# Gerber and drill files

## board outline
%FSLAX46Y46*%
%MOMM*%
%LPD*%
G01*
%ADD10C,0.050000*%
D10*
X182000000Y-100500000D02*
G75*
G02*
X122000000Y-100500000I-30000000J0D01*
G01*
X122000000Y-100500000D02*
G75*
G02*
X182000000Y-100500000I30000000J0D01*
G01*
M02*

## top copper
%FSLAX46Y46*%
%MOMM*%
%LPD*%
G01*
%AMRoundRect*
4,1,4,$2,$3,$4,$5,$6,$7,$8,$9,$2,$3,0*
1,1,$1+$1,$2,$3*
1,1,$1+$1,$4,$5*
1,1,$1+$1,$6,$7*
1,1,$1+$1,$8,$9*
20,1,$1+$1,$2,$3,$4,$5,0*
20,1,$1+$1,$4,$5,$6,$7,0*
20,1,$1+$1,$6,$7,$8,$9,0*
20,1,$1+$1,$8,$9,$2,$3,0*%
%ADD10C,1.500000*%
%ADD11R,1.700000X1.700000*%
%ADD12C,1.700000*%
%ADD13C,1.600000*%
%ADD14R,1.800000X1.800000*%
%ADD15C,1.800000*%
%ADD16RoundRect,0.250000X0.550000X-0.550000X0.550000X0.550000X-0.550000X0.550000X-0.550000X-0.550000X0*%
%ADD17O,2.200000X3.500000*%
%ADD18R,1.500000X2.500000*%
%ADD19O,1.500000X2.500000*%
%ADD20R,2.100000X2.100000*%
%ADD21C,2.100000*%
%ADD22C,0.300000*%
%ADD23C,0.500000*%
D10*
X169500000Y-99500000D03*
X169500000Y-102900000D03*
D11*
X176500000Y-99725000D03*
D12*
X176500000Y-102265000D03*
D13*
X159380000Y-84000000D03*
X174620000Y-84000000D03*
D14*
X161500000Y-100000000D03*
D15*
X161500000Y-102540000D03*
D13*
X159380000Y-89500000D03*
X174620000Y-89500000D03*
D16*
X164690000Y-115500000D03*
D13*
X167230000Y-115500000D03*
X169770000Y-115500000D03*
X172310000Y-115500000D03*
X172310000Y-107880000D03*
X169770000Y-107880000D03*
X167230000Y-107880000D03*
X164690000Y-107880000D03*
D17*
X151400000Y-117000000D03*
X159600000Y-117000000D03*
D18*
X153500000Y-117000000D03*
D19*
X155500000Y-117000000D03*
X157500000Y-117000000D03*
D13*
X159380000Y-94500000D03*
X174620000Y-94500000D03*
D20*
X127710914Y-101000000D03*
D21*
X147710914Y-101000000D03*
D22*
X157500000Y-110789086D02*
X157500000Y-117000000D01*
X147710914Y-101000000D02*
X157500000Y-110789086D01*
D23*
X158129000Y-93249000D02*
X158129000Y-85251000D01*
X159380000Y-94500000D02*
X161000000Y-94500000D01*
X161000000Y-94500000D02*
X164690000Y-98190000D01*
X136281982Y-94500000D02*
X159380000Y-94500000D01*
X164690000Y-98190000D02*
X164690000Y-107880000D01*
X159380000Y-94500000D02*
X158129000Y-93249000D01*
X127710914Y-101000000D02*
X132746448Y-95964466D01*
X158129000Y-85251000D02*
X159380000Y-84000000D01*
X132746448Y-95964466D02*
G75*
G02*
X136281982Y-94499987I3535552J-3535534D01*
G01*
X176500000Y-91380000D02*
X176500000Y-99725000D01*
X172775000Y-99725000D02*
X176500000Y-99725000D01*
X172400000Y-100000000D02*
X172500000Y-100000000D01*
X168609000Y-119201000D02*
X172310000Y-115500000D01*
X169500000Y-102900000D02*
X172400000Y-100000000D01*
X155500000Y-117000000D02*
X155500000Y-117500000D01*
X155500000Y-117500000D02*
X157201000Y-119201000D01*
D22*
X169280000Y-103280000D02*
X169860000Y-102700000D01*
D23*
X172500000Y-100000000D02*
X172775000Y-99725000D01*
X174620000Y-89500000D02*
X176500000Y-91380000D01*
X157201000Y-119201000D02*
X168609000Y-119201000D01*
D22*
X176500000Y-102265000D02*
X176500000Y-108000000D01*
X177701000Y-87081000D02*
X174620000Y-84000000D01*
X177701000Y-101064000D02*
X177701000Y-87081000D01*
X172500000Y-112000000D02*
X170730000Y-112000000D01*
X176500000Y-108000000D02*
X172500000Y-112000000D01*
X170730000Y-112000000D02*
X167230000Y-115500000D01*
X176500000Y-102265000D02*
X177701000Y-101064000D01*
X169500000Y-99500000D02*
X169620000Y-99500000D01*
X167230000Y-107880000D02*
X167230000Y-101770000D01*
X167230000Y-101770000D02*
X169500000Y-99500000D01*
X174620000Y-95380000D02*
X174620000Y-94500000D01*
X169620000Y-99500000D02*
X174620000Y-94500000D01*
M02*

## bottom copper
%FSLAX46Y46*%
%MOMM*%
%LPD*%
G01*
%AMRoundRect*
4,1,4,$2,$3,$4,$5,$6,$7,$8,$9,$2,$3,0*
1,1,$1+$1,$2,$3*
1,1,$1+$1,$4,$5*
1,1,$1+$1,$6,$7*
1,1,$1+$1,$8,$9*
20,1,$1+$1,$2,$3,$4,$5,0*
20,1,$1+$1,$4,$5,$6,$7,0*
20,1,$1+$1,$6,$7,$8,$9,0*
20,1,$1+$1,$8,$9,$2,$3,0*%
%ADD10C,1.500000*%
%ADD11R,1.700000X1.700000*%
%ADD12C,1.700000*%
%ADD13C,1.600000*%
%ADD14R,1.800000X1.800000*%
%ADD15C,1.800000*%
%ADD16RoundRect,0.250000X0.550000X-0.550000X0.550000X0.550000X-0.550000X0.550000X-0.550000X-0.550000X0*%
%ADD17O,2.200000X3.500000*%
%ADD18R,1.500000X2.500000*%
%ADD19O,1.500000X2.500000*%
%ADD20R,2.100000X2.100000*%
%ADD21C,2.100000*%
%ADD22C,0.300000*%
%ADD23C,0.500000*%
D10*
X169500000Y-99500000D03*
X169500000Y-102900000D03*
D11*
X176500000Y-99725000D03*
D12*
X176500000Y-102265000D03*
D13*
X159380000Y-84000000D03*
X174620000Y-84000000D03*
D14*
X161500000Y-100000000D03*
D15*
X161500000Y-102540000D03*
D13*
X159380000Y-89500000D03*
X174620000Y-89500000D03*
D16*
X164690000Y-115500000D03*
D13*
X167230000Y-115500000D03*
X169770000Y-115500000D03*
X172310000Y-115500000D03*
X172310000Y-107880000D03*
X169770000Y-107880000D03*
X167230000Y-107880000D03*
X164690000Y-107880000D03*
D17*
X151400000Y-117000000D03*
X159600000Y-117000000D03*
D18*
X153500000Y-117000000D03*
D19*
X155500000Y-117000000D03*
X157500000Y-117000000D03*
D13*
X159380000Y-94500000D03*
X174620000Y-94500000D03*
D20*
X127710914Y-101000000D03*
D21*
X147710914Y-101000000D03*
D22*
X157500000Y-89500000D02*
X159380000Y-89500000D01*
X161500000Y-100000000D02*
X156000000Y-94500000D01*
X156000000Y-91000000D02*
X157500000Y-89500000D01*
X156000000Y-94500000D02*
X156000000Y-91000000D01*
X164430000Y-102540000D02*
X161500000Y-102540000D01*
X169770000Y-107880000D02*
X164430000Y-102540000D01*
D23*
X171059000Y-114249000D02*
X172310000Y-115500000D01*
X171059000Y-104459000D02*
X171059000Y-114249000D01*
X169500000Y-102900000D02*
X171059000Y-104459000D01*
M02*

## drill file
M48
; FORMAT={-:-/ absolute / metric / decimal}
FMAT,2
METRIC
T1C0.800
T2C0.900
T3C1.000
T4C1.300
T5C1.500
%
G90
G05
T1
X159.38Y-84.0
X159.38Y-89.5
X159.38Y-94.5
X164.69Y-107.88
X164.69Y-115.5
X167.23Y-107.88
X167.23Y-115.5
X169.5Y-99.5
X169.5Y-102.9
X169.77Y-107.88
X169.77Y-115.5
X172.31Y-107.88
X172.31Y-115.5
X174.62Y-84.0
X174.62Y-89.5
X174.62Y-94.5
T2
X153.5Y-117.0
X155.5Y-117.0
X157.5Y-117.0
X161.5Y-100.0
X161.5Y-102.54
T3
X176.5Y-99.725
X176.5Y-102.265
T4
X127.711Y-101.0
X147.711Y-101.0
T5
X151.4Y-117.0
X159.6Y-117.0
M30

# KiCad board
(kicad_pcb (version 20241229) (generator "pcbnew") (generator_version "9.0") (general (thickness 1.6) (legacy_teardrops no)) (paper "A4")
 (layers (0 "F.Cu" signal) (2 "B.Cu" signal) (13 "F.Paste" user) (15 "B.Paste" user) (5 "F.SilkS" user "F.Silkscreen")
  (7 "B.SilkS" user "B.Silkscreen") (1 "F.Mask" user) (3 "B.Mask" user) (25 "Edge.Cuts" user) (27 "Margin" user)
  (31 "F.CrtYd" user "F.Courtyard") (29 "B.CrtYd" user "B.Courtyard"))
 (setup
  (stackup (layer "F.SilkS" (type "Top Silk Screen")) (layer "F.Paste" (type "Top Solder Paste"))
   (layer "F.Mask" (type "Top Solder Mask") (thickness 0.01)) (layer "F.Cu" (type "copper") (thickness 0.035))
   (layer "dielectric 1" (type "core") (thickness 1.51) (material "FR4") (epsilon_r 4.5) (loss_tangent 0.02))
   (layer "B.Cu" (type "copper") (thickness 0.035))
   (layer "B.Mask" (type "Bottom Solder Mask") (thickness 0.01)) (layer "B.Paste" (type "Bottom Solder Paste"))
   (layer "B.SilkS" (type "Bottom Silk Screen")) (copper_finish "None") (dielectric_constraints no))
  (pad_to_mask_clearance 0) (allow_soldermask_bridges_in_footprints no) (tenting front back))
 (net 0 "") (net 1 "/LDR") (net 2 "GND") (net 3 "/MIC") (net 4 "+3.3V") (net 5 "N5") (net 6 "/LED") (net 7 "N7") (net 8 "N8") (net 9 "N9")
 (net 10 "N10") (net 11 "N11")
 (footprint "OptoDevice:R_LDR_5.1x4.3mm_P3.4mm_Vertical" (layer "F.Cu") (at 169.5 99.5 -90)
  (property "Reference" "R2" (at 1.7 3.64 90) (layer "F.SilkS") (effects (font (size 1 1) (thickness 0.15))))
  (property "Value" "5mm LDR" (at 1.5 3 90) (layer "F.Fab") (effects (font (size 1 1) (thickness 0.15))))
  (pad "1" thru_hole circle (at 0 0 270) (size 1.5 1.5) (drill 0.8) (layers "*.Cu" "*.Mask") (remove_unused_layers no) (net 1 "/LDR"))
  (pad "2" thru_hole circle (at 3.4 0 270) (size 1.5 1.5) (drill 0.8) (layers "*.Cu" "*.Mask") (remove_unused_layers no) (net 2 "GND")))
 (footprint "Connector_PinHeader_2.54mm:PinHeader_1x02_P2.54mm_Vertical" (layer "F.Cu") (at 176.5 99.725)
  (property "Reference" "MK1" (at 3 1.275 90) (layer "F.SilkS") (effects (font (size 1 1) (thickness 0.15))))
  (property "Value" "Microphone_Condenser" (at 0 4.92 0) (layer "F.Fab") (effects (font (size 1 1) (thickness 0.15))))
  (pad "1" thru_hole rect (at 0 0) (size 1.7 1.7) (drill 1) (layers "*.Cu" "*.Mask") (remove_unused_layers no) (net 2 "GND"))
  (pad "2" thru_hole circle (at 0 2.54) (size 1.7 1.7) (drill 1) (layers "*.Cu" "*.Mask") (remove_unused_layers no) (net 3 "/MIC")))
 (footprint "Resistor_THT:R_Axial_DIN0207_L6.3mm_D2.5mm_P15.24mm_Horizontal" (layer "F.Cu") (at 159.38 84)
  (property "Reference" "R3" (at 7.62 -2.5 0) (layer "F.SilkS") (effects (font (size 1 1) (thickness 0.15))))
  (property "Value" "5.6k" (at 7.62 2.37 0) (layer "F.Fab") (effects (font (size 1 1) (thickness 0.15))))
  (pad "1" thru_hole circle (at 0 0) (size 1.6 1.6) (drill 0.8) (layers "*.Cu" "*.Mask") (remove_unused_layers no) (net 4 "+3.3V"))
  (pad "2" thru_hole circle (at 15.24 0) (size 1.6 1.6) (drill 0.8) (layers "*.Cu" "*.Mask") (remove_unused_layers no) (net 3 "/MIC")))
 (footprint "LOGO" (layer "F.Cu") (at 151.915435 78.764812)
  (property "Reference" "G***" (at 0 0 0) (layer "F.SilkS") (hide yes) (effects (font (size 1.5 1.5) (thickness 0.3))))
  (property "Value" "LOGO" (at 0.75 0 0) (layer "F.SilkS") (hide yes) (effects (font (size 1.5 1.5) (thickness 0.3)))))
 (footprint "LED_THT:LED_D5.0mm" (layer "F.Cu") (at 161.5 100 -90)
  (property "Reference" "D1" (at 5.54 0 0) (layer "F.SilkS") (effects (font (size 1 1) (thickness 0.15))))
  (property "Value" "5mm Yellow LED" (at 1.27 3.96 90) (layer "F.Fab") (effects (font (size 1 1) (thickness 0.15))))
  (pad "1" thru_hole rect (at 0 0 270) (size 1.8 1.8) (drill 0.9) (layers "*.Cu" "*.Mask") (remove_unused_layers no) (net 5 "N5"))
  (pad "2" thru_hole circle (at 2.54 0 270) (size 1.8 1.8) (drill 0.9) (layers "*.Cu" "*.Mask") (remove_unused_layers no) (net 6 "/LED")))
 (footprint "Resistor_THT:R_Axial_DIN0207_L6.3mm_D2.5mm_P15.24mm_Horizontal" (layer "F.Cu") (at 159.38 89.5)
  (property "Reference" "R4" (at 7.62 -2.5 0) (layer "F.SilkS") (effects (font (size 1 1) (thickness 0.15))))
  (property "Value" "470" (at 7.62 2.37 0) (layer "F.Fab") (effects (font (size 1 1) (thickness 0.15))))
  (pad "1" thru_hole circle (at 0 0) (size 1.6 1.6) (drill 0.8) (layers "*.Cu" "*.Mask") (remove_unused_layers no) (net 5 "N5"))
  (pad "2" thru_hole circle (at 15.24 0) (size 1.6 1.6) (drill 0.8) (layers "*.Cu" "*.Mask") (remove_unused_layers no) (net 2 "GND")))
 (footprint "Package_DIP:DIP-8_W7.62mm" (layer "F.Cu") (at 164.69 115.5 90)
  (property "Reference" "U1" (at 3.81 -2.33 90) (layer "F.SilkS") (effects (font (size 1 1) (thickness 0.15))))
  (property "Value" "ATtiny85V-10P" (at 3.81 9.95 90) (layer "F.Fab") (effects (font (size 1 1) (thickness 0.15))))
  (pad "1" thru_hole roundrect (at 0 0 90) (size 1.6 1.6) (drill 0.8) (layers "*.Cu" "*.Mask") (remove_unused_layers no)
   (roundrect_rratio 0.15625) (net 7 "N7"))
  (pad "2" thru_hole circle (at 0 2.54 90) (size 1.6 1.6) (drill 0.8) (layers "*.Cu" "*.Mask") (remove_unused_layers no) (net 3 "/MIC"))
  (pad "3" thru_hole circle (at 0 5.08 90) (size 1.6 1.6) (drill 0.8) (layers "*.Cu" "*.Mask") (remove_unused_layers no) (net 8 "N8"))
  (pad "4" thru_hole circle (at 0 7.62 90) (size 1.6 1.6) (drill 0.8) (layers "*.Cu" "*.Mask") (remove_unused_layers no) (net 2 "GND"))
  (pad "5" thru_hole circle (at 7.62 7.62 90) (size 1.6 1.6) (drill 0.8) (layers "*.Cu" "*.Mask") (remove_unused_layers no) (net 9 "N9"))
  (pad "6" thru_hole circle (at 7.62 5.08 90) (size 1.6 1.6) (drill 0.8) (layers "*.Cu" "*.Mask") (remove_unused_layers no) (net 6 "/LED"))
  (pad "7" thru_hole circle (at 7.62 2.54 90) (size 1.6 1.6) (drill 0.8) (layers "*.Cu" "*.Mask") (remove_unused_layers no) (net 1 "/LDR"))
  (pad "8" thru_hole circle (at 7.62 0 90) (size 1.6 1.6) (drill 0.8) (layers "*.Cu" "*.Mask") (remove_unused_layers no) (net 4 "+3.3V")))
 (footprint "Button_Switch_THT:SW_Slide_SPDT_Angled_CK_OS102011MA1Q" (layer "F.Cu") (at 153.5 117)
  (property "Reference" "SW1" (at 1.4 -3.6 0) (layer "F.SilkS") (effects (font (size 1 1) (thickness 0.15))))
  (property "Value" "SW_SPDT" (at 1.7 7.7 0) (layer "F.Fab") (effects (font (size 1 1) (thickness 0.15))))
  (pad "" thru_hole oval (at -2.1 0) (size 2.2 3.5) (drill 1.5) (layers "*.Cu" "*.Mask") (remove_unused_layers no))
  (pad "" thru_hole oval (at 6.1 0) (size 2.2 3.5) (drill 1.5) (layers "*.Cu" "*.Mask") (remove_unused_layers no))
  (pad "1" thru_hole rect (at 0 0) (size 1.5 2.5) (drill 0.9) (layers "*.Cu" "*.Mask") (remove_unused_layers no) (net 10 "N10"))
  (pad "2" thru_hole oval (at 2 0) (size 1.5 2.5) (drill 0.9) (layers "*.Cu" "*.Mask") (remove_unused_layers no) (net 2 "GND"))
  (pad "3" thru_hole oval (at 4 0) (size 1.5 2.5) (drill 0.9) (layers "*.Cu" "*.Mask") (remove_unused_layers no) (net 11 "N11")))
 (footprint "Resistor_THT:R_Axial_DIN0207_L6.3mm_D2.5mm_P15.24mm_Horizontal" (layer "F.Cu") (at 159.38 94.5)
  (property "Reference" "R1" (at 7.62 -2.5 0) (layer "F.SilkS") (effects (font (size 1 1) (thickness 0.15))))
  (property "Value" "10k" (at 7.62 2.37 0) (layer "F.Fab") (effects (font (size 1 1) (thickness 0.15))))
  (pad "1" thru_hole circle (at 0 0) (size 1.6 1.6) (drill 0.8) (layers "*.Cu" "*.Mask") (remove_unused_layers no) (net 4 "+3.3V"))
  (pad "2" thru_hole circle (at 15.24 0) (size 1.6 1.6) (drill 0.8) (layers "*.Cu" "*.Mask") (remove_unused_layers no) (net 1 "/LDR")))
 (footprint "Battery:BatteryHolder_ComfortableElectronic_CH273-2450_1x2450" (layer "F.Cu") (at 127.710914 101)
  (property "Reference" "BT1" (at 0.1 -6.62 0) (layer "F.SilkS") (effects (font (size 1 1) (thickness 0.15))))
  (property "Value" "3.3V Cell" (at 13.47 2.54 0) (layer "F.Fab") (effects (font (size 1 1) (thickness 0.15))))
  (pad "1" thru_hole rect (at 0 0 270) (size 2.1 2.1) (drill 1.3) (layers "*.Cu" "*.Mask") (remove_unused_layers no) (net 4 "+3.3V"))
  (pad "2" thru_hole circle (at 20 0 270) (size 2.1 2.1) (drill 1.3) (layers "*.Cu" "*.Mask") (remove_unused_layers no) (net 11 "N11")))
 (gr_circle (center 152 100.5) (end 182 100.5) (stroke (width 0.05) (type solid)) (fill no) (locked yes) (layer "Edge.Cuts"))
 (segment (start 157.5 110.789086) (end 157.5 117) (width 0.3) (layer "F.Cu") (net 11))
 (segment (start 147.710914 101) (end 157.5 110.789086) (width 0.3) (layer "F.Cu") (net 11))
 (segment (start 158.129 93.249) (end 158.129 85.251) (width 0.5) (layer "F.Cu") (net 4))
 (segment (start 159.38 94.5) (end 161 94.5) (width 0.5) (layer "F.Cu") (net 4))
 (segment (start 161 94.5) (end 164.69 98.19) (width 0.5) (layer "F.Cu") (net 4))
 (segment (start 136.281982 94.5) (end 159.38 94.5) (width 0.5) (layer "F.Cu") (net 4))
 (segment (start 164.69 98.19) (end 164.69 107.88) (width 0.5) (layer "F.Cu") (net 4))
 (segment (start 159.38 94.5) (end 158.129 93.249) (width 0.5) (layer "F.Cu") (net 4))
 (segment (start 127.710914 101) (end 132.746448 95.964466) (width 0.5) (layer "F.Cu") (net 4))
 (segment (start 158.129 85.251) (end 159.38 84) (width 0.5) (layer "F.Cu") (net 4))
 (arc (start 132.746448 95.964466) (mid 134.368565 94.880602) (end 136.281982 94.5) (width 0.5) (layer "F.Cu") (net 4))
 (segment (start 157.5 89.5) (end 159.38 89.5) (width 0.3) (layer "B.Cu") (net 5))
 (segment (start 161.5 100) (end 156 94.5) (width 0.3) (layer "B.Cu") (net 5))
 (segment (start 156 91) (end 157.5 89.5) (width 0.3) (layer "B.Cu") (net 5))
 (segment (start 156 94.5) (end 156 91) (width 0.3) (layer "B.Cu") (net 5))
 (segment (start 164.43 102.54) (end 161.5 102.54) (width 0.3) (layer "B.Cu") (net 6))
 (segment (start 169.77 107.88) (end 164.43 102.54) (width 0.3) (layer "B.Cu") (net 6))
 (segment (start 176.5 91.38) (end 176.5 99.725) (width 0.5) (layer "F.Cu") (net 2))
 (segment (start 172.775 99.725) (end 176.5 99.725) (width 0.5) (layer "F.Cu") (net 2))
 (segment (start 172.4 100) (end 172.5 100) (width 0.5) (layer "F.Cu") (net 2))
 (segment (start 168.609 119.201) (end 172.31 115.5) (width 0.5) (layer "F.Cu") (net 2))
 (segment (start 169.5 102.9) (end 172.4 100) (width 0.5) (layer "F.Cu") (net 2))
 (segment (start 155.5 117) (end 155.5 117.5) (width 0.5) (layer "F.Cu") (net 2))
 (segment (start 155.5 117.5) (end 157.201 119.201) (width 0.5) (layer "F.Cu") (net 2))
 (segment (start 169.28 103.28) (end 169.86 102.7) (width 0.3) (layer "F.Cu") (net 2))
 (segment (start 172.5 100) (end 172.775 99.725) (width 0.5) (layer "F.Cu") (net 2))
 (segment (start 174.62 89.5) (end 176.5 91.38) (width 0.5) (layer "F.Cu") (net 2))
 (segment (start 157.201 119.201) (end 168.609 119.201) (width 0.5) (layer "F.Cu") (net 2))
 (segment (start 171.059 114.249) (end 172.31 115.5) (width 0.5) (layer "B.Cu") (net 2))
 (segment (start 171.059 104.459) (end 171.059 114.249) (width 0.5) (layer "B.Cu") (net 2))
 (segment (start 169.5 102.9) (end 171.059 104.459) (width 0.5) (layer "B.Cu") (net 2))
 (segment (start 176.5 102.265) (end 176.5 108) (width 0.3) (layer "F.Cu") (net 3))
 (segment (start 177.701 87.081) (end 174.62 84) (width 0.3) (layer "F.Cu") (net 3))
 (segment (start 177.701 101.064) (end 177.701 87.081) (width 0.3) (layer "F.Cu") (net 3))
 (segment (start 172.5 112) (end 170.73 112) (width 0.3) (layer "F.Cu") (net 3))
 (segment (start 176.5 108) (end 172.5 112) (width 0.3) (layer "F.Cu") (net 3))
 (segment (start 170.73 112) (end 167.23 115.5) (width 0.3) (layer "F.Cu") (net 3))
 (segment (start 176.5 102.265) (end 177.701 101.064) (width 0.3) (layer "F.Cu") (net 3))
 (segment (start 169.5 99.5) (end 169.62 99.5) (width 0.3) (layer "F.Cu") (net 1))
 (segment (start 167.23 107.88) (end 167.23 101.77) (width 0.3) (layer "F.Cu") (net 1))
 (segment (start 167.23 101.77) (end 169.5 99.5) (width 0.3) (layer "F.Cu") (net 1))
 (segment (start 174.62 95.38) (end 174.62 94.5) (width 0.3) (layer "F.Cu") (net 1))
 (segment (start 169.62 99.5) (end 174.62 94.5) (width 0.3) (layer "F.Cu") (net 1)))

